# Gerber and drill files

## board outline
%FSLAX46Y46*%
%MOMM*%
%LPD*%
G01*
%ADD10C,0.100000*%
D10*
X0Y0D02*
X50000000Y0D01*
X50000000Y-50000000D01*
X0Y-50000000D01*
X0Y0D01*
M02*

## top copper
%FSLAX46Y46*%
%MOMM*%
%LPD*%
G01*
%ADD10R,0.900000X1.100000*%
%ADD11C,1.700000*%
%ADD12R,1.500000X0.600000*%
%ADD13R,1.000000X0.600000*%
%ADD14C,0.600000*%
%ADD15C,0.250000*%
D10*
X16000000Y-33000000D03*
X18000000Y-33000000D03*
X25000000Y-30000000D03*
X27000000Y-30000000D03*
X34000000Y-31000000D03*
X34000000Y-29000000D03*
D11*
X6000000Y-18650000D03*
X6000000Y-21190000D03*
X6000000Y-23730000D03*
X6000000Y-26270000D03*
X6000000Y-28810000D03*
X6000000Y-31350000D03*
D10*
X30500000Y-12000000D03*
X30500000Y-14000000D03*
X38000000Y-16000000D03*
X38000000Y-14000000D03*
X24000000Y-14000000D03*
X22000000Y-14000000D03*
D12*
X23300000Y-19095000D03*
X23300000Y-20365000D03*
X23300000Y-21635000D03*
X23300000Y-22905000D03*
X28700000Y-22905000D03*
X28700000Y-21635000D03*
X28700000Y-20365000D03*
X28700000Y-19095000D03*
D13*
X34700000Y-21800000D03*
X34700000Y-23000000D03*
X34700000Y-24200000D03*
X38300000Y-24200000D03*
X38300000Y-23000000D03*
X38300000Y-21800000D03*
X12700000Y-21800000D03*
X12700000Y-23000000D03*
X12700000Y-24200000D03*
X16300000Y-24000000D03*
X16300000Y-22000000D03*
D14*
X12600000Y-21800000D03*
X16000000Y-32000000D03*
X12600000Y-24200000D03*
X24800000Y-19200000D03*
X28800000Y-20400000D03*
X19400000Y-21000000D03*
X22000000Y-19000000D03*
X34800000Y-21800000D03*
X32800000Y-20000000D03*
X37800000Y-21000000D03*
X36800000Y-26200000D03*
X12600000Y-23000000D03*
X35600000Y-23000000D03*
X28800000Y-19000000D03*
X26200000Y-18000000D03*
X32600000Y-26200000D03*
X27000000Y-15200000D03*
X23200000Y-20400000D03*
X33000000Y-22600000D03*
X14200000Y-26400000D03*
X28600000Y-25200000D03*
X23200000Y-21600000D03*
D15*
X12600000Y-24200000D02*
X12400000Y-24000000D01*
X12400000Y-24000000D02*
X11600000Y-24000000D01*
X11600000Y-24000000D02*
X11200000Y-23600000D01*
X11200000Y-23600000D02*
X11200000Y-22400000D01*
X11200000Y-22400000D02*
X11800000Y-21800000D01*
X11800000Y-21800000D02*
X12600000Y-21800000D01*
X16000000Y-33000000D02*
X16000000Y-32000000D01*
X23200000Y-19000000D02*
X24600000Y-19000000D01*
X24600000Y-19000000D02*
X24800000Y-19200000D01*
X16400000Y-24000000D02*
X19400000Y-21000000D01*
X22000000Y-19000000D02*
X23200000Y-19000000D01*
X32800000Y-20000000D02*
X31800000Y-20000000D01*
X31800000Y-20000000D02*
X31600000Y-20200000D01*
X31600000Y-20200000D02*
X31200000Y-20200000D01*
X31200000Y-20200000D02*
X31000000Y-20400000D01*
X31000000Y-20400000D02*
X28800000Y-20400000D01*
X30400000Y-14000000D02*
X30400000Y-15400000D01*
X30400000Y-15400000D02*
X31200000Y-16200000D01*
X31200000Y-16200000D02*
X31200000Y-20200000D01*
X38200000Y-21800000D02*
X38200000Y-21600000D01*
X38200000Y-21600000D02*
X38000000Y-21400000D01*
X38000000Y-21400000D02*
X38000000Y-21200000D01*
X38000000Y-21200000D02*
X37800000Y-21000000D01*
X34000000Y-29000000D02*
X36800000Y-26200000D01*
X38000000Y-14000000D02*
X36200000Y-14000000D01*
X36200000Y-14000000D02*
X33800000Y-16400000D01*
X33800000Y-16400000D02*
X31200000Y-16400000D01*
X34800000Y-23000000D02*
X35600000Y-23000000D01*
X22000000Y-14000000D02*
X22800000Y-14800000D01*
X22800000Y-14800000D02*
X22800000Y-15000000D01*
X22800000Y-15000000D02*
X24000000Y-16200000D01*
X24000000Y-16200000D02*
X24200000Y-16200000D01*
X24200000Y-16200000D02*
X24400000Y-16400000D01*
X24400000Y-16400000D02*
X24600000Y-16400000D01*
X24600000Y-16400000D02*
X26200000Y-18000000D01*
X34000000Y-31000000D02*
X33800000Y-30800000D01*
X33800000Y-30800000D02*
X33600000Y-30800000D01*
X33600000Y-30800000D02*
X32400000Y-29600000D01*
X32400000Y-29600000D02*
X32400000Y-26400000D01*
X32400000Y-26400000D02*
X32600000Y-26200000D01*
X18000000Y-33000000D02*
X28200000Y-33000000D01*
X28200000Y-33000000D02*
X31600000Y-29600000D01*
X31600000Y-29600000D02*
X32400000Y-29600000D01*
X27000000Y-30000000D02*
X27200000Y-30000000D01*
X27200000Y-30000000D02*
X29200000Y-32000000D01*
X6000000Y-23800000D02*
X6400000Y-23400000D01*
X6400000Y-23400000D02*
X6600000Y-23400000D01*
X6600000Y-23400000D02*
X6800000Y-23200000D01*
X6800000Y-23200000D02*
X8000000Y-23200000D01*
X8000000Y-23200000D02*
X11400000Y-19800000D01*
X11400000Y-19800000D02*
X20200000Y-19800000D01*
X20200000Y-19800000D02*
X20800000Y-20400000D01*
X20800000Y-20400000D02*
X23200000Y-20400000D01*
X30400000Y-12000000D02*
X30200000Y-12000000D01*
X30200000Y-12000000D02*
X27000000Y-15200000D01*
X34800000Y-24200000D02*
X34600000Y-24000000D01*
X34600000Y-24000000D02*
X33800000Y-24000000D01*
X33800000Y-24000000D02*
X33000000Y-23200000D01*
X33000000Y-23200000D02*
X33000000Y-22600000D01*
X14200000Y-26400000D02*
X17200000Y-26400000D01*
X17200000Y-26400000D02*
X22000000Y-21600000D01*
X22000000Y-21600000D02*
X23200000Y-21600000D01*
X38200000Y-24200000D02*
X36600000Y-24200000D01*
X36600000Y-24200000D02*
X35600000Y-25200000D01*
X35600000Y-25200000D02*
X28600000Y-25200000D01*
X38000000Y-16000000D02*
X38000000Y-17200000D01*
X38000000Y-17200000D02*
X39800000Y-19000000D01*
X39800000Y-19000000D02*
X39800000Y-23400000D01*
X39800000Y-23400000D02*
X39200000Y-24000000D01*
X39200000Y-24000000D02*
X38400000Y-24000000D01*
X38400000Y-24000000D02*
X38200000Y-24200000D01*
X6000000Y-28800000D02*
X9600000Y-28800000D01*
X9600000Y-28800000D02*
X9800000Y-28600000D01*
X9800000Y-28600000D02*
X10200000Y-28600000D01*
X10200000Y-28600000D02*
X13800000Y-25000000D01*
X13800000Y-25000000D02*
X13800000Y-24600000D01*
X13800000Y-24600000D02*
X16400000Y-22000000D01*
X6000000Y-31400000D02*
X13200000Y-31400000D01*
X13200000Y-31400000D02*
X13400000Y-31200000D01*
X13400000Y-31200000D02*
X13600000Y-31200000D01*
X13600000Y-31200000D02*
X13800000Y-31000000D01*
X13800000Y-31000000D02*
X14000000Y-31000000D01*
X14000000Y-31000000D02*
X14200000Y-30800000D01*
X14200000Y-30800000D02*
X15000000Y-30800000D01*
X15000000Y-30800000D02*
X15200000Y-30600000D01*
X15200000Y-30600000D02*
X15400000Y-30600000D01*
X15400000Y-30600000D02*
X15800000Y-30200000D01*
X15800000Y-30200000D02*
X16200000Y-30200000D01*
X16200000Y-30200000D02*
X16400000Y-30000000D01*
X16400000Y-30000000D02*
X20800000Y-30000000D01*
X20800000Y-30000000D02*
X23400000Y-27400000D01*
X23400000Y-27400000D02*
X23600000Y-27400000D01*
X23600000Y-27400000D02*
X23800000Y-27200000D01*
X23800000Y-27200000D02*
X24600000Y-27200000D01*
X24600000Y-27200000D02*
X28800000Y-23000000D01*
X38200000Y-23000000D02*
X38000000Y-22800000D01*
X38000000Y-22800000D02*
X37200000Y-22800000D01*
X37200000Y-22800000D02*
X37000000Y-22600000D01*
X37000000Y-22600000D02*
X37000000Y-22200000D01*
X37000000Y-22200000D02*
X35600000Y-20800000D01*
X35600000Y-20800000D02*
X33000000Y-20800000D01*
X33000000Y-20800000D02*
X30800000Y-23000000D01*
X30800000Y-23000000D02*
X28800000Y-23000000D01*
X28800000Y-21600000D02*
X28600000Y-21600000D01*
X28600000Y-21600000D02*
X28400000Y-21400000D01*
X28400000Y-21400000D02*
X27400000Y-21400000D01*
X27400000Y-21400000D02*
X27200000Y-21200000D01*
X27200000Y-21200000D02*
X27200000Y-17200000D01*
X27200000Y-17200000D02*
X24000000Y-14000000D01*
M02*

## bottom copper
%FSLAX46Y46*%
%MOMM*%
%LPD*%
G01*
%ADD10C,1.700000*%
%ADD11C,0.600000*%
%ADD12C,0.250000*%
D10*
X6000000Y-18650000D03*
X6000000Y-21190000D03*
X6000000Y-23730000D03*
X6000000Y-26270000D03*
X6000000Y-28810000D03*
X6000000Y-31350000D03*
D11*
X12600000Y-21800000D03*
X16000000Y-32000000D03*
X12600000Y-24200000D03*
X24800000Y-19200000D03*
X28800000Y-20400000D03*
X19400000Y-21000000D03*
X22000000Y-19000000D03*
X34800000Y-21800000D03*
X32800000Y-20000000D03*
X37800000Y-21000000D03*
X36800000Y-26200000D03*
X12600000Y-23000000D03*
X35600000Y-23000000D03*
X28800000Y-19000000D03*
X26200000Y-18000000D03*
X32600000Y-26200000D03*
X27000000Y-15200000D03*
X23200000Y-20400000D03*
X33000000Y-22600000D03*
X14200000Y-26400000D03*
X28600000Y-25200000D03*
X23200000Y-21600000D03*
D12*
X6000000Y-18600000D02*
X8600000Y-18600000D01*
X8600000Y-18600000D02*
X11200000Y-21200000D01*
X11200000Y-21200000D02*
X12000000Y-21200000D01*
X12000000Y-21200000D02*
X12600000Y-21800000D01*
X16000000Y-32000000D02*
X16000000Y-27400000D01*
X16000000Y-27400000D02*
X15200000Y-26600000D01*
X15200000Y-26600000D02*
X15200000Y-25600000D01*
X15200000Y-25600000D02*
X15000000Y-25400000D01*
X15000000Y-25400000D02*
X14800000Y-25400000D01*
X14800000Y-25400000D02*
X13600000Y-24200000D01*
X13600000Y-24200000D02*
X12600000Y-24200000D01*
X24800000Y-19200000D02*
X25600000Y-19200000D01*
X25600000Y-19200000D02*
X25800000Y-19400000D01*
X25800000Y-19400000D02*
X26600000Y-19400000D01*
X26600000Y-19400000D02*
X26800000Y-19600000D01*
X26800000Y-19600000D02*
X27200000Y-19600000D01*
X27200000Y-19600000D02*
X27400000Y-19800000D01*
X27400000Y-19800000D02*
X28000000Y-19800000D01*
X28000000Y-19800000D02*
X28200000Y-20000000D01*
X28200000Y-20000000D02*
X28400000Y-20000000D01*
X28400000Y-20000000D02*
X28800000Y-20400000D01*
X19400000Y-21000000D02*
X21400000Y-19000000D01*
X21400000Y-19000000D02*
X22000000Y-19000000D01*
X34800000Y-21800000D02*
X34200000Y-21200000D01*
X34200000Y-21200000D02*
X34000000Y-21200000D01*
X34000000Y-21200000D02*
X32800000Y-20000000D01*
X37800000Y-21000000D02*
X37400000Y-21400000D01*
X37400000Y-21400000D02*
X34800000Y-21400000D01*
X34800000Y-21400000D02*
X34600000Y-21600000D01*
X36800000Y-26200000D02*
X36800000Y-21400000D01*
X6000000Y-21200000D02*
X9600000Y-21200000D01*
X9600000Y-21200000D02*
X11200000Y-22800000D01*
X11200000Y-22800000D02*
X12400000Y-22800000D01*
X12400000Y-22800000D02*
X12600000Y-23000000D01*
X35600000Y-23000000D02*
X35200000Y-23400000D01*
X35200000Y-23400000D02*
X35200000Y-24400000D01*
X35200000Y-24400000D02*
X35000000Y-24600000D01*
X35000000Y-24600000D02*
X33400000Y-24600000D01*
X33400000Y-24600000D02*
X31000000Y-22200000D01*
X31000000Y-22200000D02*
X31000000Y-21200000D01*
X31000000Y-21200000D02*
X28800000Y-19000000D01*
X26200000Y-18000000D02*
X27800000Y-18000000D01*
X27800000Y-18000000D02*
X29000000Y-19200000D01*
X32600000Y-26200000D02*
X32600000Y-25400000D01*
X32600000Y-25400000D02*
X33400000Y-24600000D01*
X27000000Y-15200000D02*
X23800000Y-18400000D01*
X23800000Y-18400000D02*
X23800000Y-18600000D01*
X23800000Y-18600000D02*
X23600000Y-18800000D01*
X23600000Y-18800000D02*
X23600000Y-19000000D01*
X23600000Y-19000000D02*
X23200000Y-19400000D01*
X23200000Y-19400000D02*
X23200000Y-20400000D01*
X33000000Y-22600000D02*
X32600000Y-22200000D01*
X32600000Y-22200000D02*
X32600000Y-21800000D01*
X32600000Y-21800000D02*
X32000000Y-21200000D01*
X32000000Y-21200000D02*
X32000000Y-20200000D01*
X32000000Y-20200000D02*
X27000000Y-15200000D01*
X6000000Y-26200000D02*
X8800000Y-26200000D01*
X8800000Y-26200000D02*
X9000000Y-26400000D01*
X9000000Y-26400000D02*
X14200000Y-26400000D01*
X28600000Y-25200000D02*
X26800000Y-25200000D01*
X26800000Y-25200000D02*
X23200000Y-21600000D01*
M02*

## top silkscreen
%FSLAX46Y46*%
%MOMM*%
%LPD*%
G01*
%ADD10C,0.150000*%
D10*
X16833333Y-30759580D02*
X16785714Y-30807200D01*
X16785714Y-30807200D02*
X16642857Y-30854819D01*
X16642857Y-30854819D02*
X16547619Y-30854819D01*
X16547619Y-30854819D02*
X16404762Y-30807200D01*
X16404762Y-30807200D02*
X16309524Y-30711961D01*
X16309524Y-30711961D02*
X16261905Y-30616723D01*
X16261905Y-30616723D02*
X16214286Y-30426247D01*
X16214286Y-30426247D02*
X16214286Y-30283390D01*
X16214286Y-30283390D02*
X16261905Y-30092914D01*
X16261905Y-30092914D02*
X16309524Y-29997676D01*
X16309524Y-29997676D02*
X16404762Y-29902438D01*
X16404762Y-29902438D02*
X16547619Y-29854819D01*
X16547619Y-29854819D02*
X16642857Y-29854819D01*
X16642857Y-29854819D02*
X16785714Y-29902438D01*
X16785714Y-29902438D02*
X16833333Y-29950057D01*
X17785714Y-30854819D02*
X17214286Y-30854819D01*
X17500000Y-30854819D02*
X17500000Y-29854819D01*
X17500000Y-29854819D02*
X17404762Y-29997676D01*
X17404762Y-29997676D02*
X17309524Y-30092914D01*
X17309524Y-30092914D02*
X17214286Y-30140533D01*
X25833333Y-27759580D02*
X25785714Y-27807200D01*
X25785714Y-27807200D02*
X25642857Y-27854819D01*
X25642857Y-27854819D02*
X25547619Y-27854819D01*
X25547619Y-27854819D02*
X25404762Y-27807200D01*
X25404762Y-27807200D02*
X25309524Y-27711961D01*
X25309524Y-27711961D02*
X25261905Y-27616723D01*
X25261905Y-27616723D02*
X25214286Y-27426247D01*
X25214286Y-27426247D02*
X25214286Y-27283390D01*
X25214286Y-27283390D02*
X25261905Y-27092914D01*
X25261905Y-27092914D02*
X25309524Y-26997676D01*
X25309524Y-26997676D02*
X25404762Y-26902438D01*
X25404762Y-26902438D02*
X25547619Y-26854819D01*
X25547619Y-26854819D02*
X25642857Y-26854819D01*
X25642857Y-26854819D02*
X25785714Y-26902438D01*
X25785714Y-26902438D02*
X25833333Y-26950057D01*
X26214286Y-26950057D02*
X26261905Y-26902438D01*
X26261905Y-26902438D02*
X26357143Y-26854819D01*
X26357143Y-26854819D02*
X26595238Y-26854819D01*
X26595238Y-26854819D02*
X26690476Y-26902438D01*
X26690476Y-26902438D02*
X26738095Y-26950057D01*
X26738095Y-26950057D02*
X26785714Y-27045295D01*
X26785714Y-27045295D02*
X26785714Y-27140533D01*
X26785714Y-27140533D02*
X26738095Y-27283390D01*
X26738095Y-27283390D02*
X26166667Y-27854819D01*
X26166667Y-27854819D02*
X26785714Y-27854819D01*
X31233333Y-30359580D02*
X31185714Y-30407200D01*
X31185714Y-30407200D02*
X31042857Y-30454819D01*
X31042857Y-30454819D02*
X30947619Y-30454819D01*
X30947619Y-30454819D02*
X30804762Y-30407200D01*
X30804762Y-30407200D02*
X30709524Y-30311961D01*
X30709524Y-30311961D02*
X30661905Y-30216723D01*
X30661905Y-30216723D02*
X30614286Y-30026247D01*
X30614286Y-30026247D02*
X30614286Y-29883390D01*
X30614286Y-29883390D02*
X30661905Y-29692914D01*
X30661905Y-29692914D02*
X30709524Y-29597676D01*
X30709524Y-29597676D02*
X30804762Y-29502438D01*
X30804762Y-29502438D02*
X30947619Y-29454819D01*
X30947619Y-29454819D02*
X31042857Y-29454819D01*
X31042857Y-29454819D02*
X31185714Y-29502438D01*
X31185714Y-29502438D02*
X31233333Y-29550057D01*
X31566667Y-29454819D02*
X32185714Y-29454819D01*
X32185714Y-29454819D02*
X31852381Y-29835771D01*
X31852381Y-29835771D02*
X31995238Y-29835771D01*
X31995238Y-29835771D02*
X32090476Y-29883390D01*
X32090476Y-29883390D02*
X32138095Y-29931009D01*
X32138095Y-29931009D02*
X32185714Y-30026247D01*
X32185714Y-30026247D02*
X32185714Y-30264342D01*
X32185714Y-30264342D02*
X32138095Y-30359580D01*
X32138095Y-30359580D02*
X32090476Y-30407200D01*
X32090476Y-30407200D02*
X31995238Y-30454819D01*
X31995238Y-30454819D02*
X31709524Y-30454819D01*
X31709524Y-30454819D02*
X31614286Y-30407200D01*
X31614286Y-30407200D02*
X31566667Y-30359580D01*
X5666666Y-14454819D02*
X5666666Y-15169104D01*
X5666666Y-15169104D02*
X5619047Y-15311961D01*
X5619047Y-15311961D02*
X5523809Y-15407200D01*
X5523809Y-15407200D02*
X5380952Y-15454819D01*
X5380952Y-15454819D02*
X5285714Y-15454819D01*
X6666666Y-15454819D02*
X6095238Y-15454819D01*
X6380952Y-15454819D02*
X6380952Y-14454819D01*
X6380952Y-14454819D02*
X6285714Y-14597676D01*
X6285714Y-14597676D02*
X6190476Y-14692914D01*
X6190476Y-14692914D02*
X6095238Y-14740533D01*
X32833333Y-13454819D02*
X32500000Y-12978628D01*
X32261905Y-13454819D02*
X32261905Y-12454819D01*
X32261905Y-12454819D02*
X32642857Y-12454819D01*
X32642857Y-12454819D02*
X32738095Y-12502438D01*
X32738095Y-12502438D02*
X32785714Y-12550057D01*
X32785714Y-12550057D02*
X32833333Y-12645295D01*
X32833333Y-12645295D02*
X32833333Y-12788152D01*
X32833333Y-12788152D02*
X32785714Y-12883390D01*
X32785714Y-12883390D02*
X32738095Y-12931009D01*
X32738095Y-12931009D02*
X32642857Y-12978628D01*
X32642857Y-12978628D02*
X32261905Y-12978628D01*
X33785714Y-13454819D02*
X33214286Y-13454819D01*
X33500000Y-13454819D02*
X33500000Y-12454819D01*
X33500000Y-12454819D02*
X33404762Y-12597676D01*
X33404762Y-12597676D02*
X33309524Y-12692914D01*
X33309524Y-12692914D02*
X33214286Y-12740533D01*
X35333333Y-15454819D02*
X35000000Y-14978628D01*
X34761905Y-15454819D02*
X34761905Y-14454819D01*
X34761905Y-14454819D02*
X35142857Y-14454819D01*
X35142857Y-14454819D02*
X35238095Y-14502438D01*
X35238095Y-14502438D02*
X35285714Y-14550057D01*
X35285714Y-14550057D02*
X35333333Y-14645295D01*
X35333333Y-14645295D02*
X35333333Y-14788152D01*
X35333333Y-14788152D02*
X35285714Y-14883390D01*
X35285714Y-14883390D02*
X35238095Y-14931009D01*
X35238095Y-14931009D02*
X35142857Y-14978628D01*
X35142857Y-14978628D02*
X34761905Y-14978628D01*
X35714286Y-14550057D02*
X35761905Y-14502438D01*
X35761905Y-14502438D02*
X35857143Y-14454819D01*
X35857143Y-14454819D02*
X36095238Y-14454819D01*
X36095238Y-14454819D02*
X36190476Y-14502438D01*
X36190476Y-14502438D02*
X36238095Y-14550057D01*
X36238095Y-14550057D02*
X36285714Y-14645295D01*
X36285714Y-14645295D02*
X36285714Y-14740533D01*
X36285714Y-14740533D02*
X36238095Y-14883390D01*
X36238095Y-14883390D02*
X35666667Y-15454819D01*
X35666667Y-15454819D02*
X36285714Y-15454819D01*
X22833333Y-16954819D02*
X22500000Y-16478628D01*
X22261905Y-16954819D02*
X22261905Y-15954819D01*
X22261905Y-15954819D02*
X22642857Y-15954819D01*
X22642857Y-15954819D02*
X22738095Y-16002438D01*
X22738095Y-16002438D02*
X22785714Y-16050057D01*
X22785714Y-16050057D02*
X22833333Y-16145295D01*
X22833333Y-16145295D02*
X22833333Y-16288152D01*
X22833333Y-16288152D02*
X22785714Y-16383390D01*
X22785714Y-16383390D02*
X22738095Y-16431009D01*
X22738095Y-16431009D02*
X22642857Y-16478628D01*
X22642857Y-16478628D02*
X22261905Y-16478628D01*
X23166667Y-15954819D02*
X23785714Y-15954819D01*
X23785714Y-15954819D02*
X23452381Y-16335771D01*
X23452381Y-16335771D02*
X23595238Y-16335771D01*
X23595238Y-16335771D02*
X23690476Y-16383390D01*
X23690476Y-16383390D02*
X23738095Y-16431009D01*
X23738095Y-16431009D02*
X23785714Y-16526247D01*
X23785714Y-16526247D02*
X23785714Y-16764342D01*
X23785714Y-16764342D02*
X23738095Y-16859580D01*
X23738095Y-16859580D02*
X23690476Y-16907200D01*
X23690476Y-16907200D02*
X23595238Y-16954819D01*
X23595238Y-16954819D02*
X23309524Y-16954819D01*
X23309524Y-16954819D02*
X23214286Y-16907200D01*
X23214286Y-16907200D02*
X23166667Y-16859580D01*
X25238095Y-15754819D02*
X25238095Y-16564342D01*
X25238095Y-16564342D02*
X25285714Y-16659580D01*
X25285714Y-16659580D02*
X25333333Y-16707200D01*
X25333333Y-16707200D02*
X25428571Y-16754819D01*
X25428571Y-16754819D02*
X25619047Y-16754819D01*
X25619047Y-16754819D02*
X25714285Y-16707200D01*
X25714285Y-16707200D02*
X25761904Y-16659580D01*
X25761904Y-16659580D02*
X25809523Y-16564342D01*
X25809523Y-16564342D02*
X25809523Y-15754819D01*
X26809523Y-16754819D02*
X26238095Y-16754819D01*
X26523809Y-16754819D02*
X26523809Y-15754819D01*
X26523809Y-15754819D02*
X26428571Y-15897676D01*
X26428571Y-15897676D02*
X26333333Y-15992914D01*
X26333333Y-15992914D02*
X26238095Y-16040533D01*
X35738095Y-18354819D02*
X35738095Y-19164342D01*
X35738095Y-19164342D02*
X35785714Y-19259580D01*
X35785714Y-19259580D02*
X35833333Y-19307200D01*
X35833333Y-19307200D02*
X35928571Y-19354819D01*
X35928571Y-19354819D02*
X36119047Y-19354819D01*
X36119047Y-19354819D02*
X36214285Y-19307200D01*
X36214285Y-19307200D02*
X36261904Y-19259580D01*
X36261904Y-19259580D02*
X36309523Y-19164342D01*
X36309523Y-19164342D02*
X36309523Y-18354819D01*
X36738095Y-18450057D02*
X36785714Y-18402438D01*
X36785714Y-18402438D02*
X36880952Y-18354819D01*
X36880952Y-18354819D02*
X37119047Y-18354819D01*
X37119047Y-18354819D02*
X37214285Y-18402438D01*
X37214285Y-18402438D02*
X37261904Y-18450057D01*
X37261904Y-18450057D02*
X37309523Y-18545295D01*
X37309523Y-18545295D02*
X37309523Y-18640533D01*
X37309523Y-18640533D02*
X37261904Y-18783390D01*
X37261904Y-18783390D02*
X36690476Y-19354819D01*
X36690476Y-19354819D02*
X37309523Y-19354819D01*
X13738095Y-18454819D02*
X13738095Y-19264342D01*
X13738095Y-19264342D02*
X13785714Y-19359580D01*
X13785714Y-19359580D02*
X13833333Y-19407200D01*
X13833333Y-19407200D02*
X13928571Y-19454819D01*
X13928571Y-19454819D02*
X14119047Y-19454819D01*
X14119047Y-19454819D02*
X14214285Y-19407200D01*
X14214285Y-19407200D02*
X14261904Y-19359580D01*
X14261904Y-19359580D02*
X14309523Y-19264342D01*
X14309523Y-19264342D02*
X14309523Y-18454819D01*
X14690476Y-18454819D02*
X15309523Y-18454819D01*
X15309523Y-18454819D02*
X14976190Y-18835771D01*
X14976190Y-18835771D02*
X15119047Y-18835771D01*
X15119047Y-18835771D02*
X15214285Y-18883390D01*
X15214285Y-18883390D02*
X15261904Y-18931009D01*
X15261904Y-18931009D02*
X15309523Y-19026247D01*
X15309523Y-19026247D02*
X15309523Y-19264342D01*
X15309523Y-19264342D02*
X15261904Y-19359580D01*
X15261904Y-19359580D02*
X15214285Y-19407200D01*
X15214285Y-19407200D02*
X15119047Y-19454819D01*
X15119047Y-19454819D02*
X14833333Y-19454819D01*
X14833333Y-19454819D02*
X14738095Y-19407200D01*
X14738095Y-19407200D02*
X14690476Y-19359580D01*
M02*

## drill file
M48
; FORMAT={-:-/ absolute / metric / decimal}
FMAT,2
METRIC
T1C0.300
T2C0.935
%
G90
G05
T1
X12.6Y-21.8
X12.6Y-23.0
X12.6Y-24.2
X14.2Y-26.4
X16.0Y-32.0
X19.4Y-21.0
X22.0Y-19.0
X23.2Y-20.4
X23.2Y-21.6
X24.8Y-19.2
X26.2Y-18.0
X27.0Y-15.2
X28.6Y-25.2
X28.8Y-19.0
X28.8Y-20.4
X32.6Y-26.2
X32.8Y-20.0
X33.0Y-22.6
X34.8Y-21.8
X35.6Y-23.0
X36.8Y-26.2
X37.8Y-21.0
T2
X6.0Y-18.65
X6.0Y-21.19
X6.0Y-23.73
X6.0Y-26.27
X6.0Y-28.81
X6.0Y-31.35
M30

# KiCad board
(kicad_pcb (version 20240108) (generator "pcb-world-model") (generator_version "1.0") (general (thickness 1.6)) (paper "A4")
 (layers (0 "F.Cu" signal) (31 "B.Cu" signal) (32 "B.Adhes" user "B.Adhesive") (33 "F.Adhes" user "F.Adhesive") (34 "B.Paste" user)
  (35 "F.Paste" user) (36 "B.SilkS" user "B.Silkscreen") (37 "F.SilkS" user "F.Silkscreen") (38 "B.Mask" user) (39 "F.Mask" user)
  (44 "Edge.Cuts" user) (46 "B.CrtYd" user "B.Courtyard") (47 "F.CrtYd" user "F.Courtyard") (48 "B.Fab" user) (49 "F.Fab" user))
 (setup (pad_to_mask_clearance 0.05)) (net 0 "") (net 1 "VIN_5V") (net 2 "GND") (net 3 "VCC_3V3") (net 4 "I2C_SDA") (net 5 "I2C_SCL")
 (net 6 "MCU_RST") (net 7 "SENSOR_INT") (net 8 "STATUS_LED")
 (gr_rect (start 0.0 0.0) (end 50.0000 50.0000) (stroke (width 0.1) (type default)) (fill none) (layer "Edge.Cuts"))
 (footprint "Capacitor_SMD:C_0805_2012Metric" (layer "F.Cu") (at 17.0000 33.0000 0)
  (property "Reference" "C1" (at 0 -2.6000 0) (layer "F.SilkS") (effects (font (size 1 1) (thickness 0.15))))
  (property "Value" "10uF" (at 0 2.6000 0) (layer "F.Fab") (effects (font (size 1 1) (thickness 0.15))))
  (pad "1" smd rect (at -1.0000 0.0000) (size 0.9000 1.1000) (layers "F.Cu" "F.Paste" "F.Mask") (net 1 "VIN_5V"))
  (pad "2" smd rect (at 1.0000 0.0000) (size 0.9000 1.1000) (layers "F.Cu" "F.Paste" "F.Mask") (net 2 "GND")))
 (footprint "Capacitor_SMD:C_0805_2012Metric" (layer "F.Cu") (at 26.0000 30.0000 0)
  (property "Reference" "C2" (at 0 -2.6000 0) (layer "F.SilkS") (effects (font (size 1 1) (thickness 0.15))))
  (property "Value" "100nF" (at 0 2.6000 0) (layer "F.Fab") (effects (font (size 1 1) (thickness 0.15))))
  (pad "1" smd rect (at -1.0000 0.0000) (size 0.9000 1.1000) (layers "F.Cu" "F.Paste" "F.Mask") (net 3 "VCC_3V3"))
  (pad "2" smd rect (at 1.0000 0.0000) (size 0.9000 1.1000) (layers "F.Cu" "F.Paste" "F.Mask") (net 2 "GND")))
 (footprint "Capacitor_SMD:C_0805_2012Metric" (layer "F.Cu") (at 34.0000 30.0000 90)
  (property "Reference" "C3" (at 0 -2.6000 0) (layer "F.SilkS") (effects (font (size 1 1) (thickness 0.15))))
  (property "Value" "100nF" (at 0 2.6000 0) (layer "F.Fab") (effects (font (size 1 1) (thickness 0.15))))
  (pad "1" smd rect (at -1.0000 0.0000) (size 0.9000 1.1000) (layers "F.Cu" "F.Paste" "F.Mask") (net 3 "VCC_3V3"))
  (pad "2" smd rect (at 1.0000 0.0000) (size 0.9000 1.1000) (layers "F.Cu" "F.Paste" "F.Mask") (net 2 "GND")))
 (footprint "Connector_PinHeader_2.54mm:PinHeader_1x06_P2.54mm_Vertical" (layer "F.Cu") (at 6.0000 25.0000 0) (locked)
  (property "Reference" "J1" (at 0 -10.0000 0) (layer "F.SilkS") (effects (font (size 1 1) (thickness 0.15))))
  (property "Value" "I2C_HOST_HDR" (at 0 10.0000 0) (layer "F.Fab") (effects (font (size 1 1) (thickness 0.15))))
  (pad "1" thru_hole circle (at 0.0000 -6.3500) (size 1.7000 1.7000) (drill 0.9350) (layers "*.Cu" "*.Mask") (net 1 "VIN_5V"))
  (pad "2" thru_hole circle (at 0.0000 -3.8100) (size 1.7000 1.7000) (drill 0.9350) (layers "*.Cu" "*.Mask") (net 2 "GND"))
  (pad "3" thru_hole circle (at 0.0000 -1.2700) (size 1.7000 1.7000) (drill 0.9350) (layers "*.Cu" "*.Mask") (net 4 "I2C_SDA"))
  (pad "4" thru_hole circle (at 0.0000 1.2700) (size 1.7000 1.7000) (drill 0.9350) (layers "*.Cu" "*.Mask") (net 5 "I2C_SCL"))
  (pad "5" thru_hole circle (at 0.0000 3.8100) (size 1.7000 1.7000) (drill 0.9350) (layers "*.Cu" "*.Mask") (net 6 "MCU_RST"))
  (pad "6" thru_hole circle (at 0.0000 6.3500) (size 1.7000 1.7000) (drill 0.9350) (layers "*.Cu" "*.Mask") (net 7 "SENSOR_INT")))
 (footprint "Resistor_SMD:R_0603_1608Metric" (layer "F.Cu") (at 30.5000 13.0000 270)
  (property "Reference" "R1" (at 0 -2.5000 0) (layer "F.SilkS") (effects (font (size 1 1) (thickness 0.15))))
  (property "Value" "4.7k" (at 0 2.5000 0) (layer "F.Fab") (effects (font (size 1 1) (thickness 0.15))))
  (pad "1" smd rect (at -1.0000 0.0000) (size 0.9000 1.1000) (layers "F.Cu" "F.Paste" "F.Mask") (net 3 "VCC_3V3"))
  (pad "2" smd rect (at 1.0000 0.0000) (size 0.9000 1.1000) (layers "F.Cu" "F.Paste" "F.Mask") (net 4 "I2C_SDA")))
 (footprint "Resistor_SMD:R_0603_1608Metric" (layer "F.Cu") (at 38.0000 15.0000 90)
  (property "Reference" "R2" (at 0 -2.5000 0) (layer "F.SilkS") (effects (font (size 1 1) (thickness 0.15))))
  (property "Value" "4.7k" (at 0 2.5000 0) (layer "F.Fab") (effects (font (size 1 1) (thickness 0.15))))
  (pad "1" smd rect (at -1.0000 0.0000) (size 0.9000 1.1000) (layers "F.Cu" "F.Paste" "F.Mask") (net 3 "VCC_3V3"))
  (pad "2" smd rect (at 1.0000 0.0000) (size 0.9000 1.1000) (layers "F.Cu" "F.Paste" "F.Mask") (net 5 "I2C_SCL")))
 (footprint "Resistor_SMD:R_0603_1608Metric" (layer "F.Cu") (at 23.0000 14.0000 180)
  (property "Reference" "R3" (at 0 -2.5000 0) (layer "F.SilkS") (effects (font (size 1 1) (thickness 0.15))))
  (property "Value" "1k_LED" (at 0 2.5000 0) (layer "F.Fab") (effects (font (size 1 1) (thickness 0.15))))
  (pad "1" smd rect (at -1.0000 0.0000) (size 0.9000 1.1000) (layers "F.Cu" "F.Paste" "F.Mask") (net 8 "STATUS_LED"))
  (pad "2" smd rect (at 1.0000 0.0000) (size 0.9000 1.1000) (layers "F.Cu" "F.Paste" "F.Mask") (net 2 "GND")))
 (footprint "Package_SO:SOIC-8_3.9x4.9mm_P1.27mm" (layer "F.Cu") (at 26.0000 21.0000 0)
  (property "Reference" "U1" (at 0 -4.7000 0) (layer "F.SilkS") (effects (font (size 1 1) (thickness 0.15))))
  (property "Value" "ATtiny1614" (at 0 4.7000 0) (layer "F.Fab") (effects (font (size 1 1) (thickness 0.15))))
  (pad "1" smd rect (at -2.7000 -1.9050) (size 1.5000 0.6000) (layers "F.Cu" "F.Paste" "F.Mask") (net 3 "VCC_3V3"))
  (pad "2" smd rect (at -2.7000 -0.6350) (size 1.5000 0.6000) (layers "F.Cu" "F.Paste" "F.Mask") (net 4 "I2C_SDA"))
  (pad "3" smd rect (at -2.7000 0.6350) (size 1.5000 0.6000) (layers "F.Cu" "F.Paste" "F.Mask") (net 5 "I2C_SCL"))
  (pad "4" smd rect (at -2.7000 1.9050) (size 1.5000 0.6000) (layers "F.Cu" "F.Paste" "F.Mask") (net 6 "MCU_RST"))
  (pad "5" smd rect (at 2.7000 1.9050) (size 1.5000 0.6000) (layers "F.Cu" "F.Paste" "F.Mask") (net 7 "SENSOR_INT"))
  (pad "6" smd rect (at 2.7000 0.6350) (size 1.5000 0.6000) (layers "F.Cu" "F.Paste" "F.Mask") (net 8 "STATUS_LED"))
  (pad "7" smd rect (at 2.7000 -0.6350) (size 1.5000 0.6000) (layers "F.Cu" "F.Paste" "F.Mask") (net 3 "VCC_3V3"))
  (pad "8" smd rect (at 2.7000 -1.9050) (size 1.5000 0.6000) (layers "F.Cu" "F.Paste" "F.Mask") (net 2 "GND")))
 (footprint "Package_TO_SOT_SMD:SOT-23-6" (layer "F.Cu") (at 36.5000 23.0000 0)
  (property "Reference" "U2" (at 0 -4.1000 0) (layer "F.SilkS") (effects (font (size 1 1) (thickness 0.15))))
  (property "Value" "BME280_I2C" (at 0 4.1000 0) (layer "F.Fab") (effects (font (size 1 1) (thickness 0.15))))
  (pad "1" smd rect (at -1.8000 -1.2000) (size 1.0000 0.6000) (layers "F.Cu" "F.Paste" "F.Mask") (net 3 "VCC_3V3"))
  (pad "2" smd rect (at -1.8000 0.0000) (size 1.0000 0.6000) (layers "F.Cu" "F.Paste" "F.Mask") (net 2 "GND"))
  (pad "3" smd rect (at -1.8000 1.2000) (size 1.0000 0.6000) (layers "F.Cu" "F.Paste" "F.Mask") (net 4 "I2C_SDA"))
  (pad "4" smd rect (at 1.8000 1.2000) (size 1.0000 0.6000) (layers "F.Cu" "F.Paste" "F.Mask") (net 5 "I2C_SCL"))
  (pad "5" smd rect (at 1.8000 0.0000) (size 1.0000 0.6000) (layers "F.Cu" "F.Paste" "F.Mask") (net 7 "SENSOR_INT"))
  (pad "6" smd rect (at 1.8000 -1.2000) (size 1.0000 0.6000) (layers "F.Cu" "F.Paste" "F.Mask") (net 3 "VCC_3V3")))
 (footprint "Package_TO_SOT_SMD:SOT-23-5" (layer "F.Cu") (at 14.5000 23.0000 0)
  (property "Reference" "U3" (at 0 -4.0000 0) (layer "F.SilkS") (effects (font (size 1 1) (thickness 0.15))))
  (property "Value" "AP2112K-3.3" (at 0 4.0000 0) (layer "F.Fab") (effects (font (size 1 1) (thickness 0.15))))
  (pad "1" smd rect (at -1.8000 -1.2000) (size 1.0000 0.6000) (layers "F.Cu" "F.Paste" "F.Mask") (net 1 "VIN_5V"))
  (pad "2" smd rect (at -1.8000 0.0000) (size 1.0000 0.6000) (layers "F.Cu" "F.Paste" "F.Mask") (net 2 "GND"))
  (pad "3" smd rect (at -1.8000 1.2000) (size 1.0000 0.6000) (layers "F.Cu" "F.Paste" "F.Mask") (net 1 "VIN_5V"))
  (pad "4" smd rect (at 1.8000 1.0000) (size 1.0000 0.6000) (layers "F.Cu" "F.Paste" "F.Mask") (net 3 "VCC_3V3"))
  (pad "5" smd rect (at 1.8000 -1.0000) (size 1.0000 0.6000) (layers "F.Cu" "F.Paste" "F.Mask") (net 6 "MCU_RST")))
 (segment (start 6.0000 18.6000) (end 8.6000 18.6000) (width 0.2500) (layer "B.Cu") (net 1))
 (segment (start 8.6000 18.6000) (end 11.2000 21.2000) (width 0.2500) (layer "B.Cu") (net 1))
 (segment (start 11.2000 21.2000) (end 12.0000 21.2000) (width 0.2500) (layer "B.Cu") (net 1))
 (segment (start 12.0000 21.2000) (end 12.6000 21.8000) (width 0.2500) (layer "B.Cu") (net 1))
 (segment (start 12.6000 24.2000) (end 12.4000 24.0000) (width 0.2500) (layer "F.Cu") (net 1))
 (segment (start 12.4000 24.0000) (end 11.6000 24.0000) (width 0.2500) (layer "F.Cu") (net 1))
 (segment (start 11.6000 24.0000) (end 11.2000 23.6000) (width 0.2500) (layer "F.Cu") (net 1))
 (segment (start 11.2000 23.6000) (end 11.2000 22.4000) (width 0.2500) (layer "F.Cu") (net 1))
 (segment (start 11.2000 22.4000) (end 11.8000 21.8000) (width 0.2500) (layer "F.Cu") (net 1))
 (segment (start 11.8000 21.8000) (end 12.6000 21.8000) (width 0.2500) (layer "F.Cu") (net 1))
 (segment (start 16.0000 33.0000) (end 16.0000 32.0000) (width 0.2500) (layer "F.Cu") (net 1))
 (segment (start 16.0000 32.0000) (end 16.0000 27.4000) (width 0.2500) (layer "B.Cu") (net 1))
 (segment (start 16.0000 27.4000) (end 15.2000 26.6000) (width 0.2500) (layer "B.Cu") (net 1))
 (segment (start 15.2000 26.6000) (end 15.2000 25.6000) (width 0.2500) (layer "B.Cu") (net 1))
 (segment (start 15.2000 25.6000) (end 15.0000 25.4000) (width 0.2500) (layer "B.Cu") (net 1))
 (segment (start 15.0000 25.4000) (end 14.8000 25.4000) (width 0.2500) (layer "B.Cu") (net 1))
 (segment (start 14.8000 25.4000) (end 13.6000 24.2000) (width 0.2500) (layer "B.Cu") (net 1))
 (segment (start 13.6000 24.2000) (end 12.6000 24.2000) (width 0.2500) (layer "B.Cu") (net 1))
 (segment (start 23.2000 19.0000) (end 24.6000 19.0000) (width 0.2500) (layer "F.Cu") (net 3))
 (segment (start 24.6000 19.0000) (end 24.8000 19.2000) (width 0.2500) (layer "F.Cu") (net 3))
 (segment (start 24.8000 19.2000) (end 25.6000 19.2000) (width 0.2500) (layer "B.Cu") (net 3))
 (segment (start 25.6000 19.2000) (end 25.8000 19.4000) (width 0.2500) (layer "B.Cu") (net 3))
 (segment (start 25.8000 19.4000) (end 26.6000 19.4000) (width 0.2500) (layer "B.Cu") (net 3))
 (segment (start 26.6000 19.4000) (end 26.8000 19.6000) (width 0.2500) (layer "B.Cu") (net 3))
 (segment (start 26.8000 19.6000) (end 27.2000 19.6000) (width 0.2500) (layer "B.Cu") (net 3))
 (segment (start 27.2000 19.6000) (end 27.4000 19.8000) (width 0.2500) (layer "B.Cu") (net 3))
 (segment (start 27.4000 19.8000) (end 28.0000 19.8000) (width 0.2500) (layer "B.Cu") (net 3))
 (segment (start 28.0000 19.8000) (end 28.2000 20.0000) (width 0.2500) (layer "B.Cu") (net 3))
 (segment (start 28.2000 20.0000) (end 28.4000 20.0000) (width 0.2500) (layer "B.Cu") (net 3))
 (segment (start 28.4000 20.0000) (end 28.8000 20.4000) (width 0.2500) (layer "B.Cu") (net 3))
 (segment (start 16.4000 24.0000) (end 19.4000 21.0000) (width 0.2500) (layer "F.Cu") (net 3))
 (segment (start 19.4000 21.0000) (end 21.4000 19.0000) (width 0.2500) (layer "B.Cu") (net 3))
 (segment (start 21.4000 19.0000) (end 22.0000 19.0000) (width 0.2500) (layer "B.Cu") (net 3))
 (segment (start 22.0000 19.0000) (end 23.2000 19.0000) (width 0.2500) (layer "F.Cu") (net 3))
 (segment (start 34.8000 21.8000) (end 34.2000 21.2000) (width 0.2500) (layer "B.Cu") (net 3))
 (segment (start 34.2000 21.2000) (end 34.0000 21.2000) (width 0.2500) (layer "B.Cu") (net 3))
 (segment (start 34.0000 21.2000) (end 32.8000 20.0000) (width 0.2500) (layer "B.Cu") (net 3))
 (segment (start 32.8000 20.0000) (end 31.8000 20.0000) (width 0.2500) (layer "F.Cu") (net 3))
 (segment (start 31.8000 20.0000) (end 31.6000 20.2000) (width 0.2500) (layer "F.Cu") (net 3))
 (segment (start 31.6000 20.2000) (end 31.2000 20.2000) (width 0.2500) (layer "F.Cu") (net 3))
 (segment (start 31.2000 20.2000) (end 31.0000 20.4000) (width 0.2500) (layer "F.Cu") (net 3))
 (segment (start 31.0000 20.4000) (end 28.8000 20.4000) (width 0.2500) (layer "F.Cu") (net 3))
 (segment (start 30.4000 14.0000) (end 30.4000 15.4000) (width 0.2500) (layer "F.Cu") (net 3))
 (segment (start 30.4000 15.4000) (end 31.2000 16.2000) (width 0.2500) (layer "F.Cu") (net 3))
 (segment (start 31.2000 16.2000) (end 31.2000 20.2000) (width 0.2500) (layer "F.Cu") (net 3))
 (segment (start 38.2000 21.8000) (end 38.2000 21.6000) (width 0.2500) (layer "F.Cu") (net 3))
 (segment (start 38.2000 21.6000) (end 38.0000 21.4000) (width 0.2500) (layer "F.Cu") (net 3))
 (segment (start 38.0000 21.4000) (end 38.0000 21.2000) (width 0.2500) (layer "F.Cu") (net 3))
 (segment (start 38.0000 21.2000) (end 37.8000 21.0000) (width 0.2500) (layer "F.Cu") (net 3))
 (segment (start 37.8000 21.0000) (end 37.4000 21.4000) (width 0.2500) (layer "B.Cu") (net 3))
 (segment (start 37.4000 21.4000) (end 34.8000 21.4000) (width 0.2500) (layer "B.Cu") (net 3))
 (segment (start 34.8000 21.4000) (end 34.6000 21.6000) (width 0.2500) (layer "B.Cu") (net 3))
 (segment (start 34.0000 29.0000) (end 36.8000 26.2000) (width 0.2500) (layer "F.Cu") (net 3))
 (segment (start 36.8000 26.2000) (end 36.8000 21.4000) (width 0.2500) (layer "B.Cu") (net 3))
 (segment (start 38.0000 14.0000) (end 36.2000 14.0000) (width 0.2500) (layer "F.Cu") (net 3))
 (segment (start 36.2000 14.0000) (end 33.8000 16.4000) (width 0.2500) (layer "F.Cu") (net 3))
 (segment (start 33.8000 16.4000) (end 31.2000 16.4000) (width 0.2500) (layer "F.Cu") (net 3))
 (segment (start 6.0000 21.2000) (end 9.6000 21.2000) (width 0.2500) (layer "B.Cu") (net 2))
 (segment (start 9.6000 21.2000) (end 11.2000 22.8000) (width 0.2500) (layer "B.Cu") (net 2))
 (segment (start 11.2000 22.8000) (end 12.4000 22.8000) (width 0.2500) (layer "B.Cu") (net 2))
 (segment (start 12.4000 22.8000) (end 12.6000 23.0000) (width 0.2500) (layer "B.Cu") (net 2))
 (segment (start 34.8000 23.0000) (end 35.6000 23.0000) (width 0.2500) (layer "F.Cu") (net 2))
 (segment (start 35.6000 23.0000) (end 35.2000 23.4000) (width 0.2500) (layer "B.Cu") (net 2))
 (segment (start 35.2000 23.4000) (end 35.2000 24.4000) (width 0.2500) (layer "B.Cu") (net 2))
 (segment (start 35.2000 24.4000) (end 35.0000 24.6000) (width 0.2500) (layer "B.Cu") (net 2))
 (segment (start 35.0000 24.6000) (end 33.4000 24.6000) (width 0.2500) (layer "B.Cu") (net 2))
 (segment (start 33.4000 24.6000) (end 31.0000 22.2000) (width 0.2500) (layer "B.Cu") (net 2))
 (segment (start 31.0000 22.2000) (end 31.0000 21.2000) (width 0.2500) (layer "B.Cu") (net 2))
 (segment (start 31.0000 21.2000) (end 28.8000 19.0000) (width 0.2500) (layer "B.Cu") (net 2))
 (segment (start 22.0000 14.0000) (end 22.8000 14.8000) (width 0.2500) (layer "F.Cu") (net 2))
 (segment (start 22.8000 14.8000) (end 22.8000 15.0000) (width 0.2500) (layer "F.Cu") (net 2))
 (segment (start 22.8000 15.0000) (end 24.0000 16.2000) (width 0.2500) (layer "F.Cu") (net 2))
 (segment (start 24.0000 16.2000) (end 24.2000 16.2000) (width 0.2500) (layer "F.Cu") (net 2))
 (segment (start 24.2000 16.2000) (end 24.4000 16.4000) (width 0.2500) (layer "F.Cu") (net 2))
 (segment (start 24.4000 16.4000) (end 24.6000 16.4000) (width 0.2500) (layer "F.Cu") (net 2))
 (segment (start 24.6000 16.4000) (end 26.2000 18.0000) (width 0.2500) (layer "F.Cu") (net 2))
 (segment (start 26.2000 18.0000) (end 27.8000 18.0000) (width 0.2500) (layer "B.Cu") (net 2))
 (segment (start 27.8000 18.0000) (end 29.0000 19.2000) (width 0.2500) (layer "B.Cu") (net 2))
 (segment (start 34.0000 31.0000) (end 33.8000 30.8000) (width 0.2500) (layer "F.Cu") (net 2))
 (segment (start 33.8000 30.8000) (end 33.6000 30.8000) (width 0.2500) (layer "F.Cu") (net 2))
 (segment (start 33.6000 30.8000) (end 32.4000 29.6000) (width 0.2500) (layer "F.Cu") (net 2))
 (segment (start 32.4000 29.6000) (end 32.4000 26.4000) (width 0.2500) (layer "F.Cu") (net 2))
 (segment (start 32.4000 26.4000) (end 32.6000 26.2000) (width 0.2500) (layer "F.Cu") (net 2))
 (segment (start 32.6000 26.2000) (end 32.6000 25.4000) (width 0.2500) (layer "B.Cu") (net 2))
 (segment (start 32.6000 25.4000) (end 33.4000 24.6000) (width 0.2500) (layer "B.Cu") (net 2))
 (segment (start 18.0000 33.0000) (end 28.2000 33.0000) (width 0.2500) (layer "F.Cu") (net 2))
 (segment (start 28.2000 33.0000) (end 31.6000 29.6000) (width 0.2500) (layer "F.Cu") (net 2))
 (segment (start 31.6000 29.6000) (end 32.4000 29.6000) (width 0.2500) (layer "F.Cu") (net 2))
 (segment (start 27.0000 30.0000) (end 27.2000 30.0000) (width 0.2500) (layer "F.Cu") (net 2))
 (segment (start 27.2000 30.0000) (end 29.2000 32.0000) (width 0.2500) (layer "F.Cu") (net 2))
 (segment (start 6.0000 23.8000) (end 6.4000 23.4000) (width 0.2500) (layer "F.Cu") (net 4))
 (segment (start 6.4000 23.4000) (end 6.6000 23.4000) (width 0.2500) (layer "F.Cu") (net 4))
 (segment (start 6.6000 23.4000) (end 6.8000 23.2000) (width 0.2500) (layer "F.Cu") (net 4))
 (segment (start 6.8000 23.2000) (end 8.0000 23.2000) (width 0.2500) (layer "F.Cu") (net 4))
 (segment (start 8.0000 23.2000) (end 11.4000 19.8000) (width 0.2500) (layer "F.Cu") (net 4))
 (segment (start 11.4000 19.8000) (end 20.2000 19.8000) (width 0.2500) (layer "F.Cu") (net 4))
 (segment (start 20.2000 19.8000) (end 20.8000 20.4000) (width 0.2500) (layer "F.Cu") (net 4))
 (segment (start 20.8000 20.4000) (end 23.2000 20.4000) (width 0.2500) (layer "F.Cu") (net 4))
 (segment (start 30.4000 12.0000) (end 30.2000 12.0000) (width 0.2500) (layer "F.Cu") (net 4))
 (segment (start 30.2000 12.0000) (end 27.0000 15.2000) (width 0.2500) (layer "F.Cu") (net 4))
 (segment (start 27.0000 15.2000) (end 23.8000 18.4000) (width 0.2500) (layer "B.Cu") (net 4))
 (segment (start 23.8000 18.4000) (end 23.8000 18.6000) (width 0.2500) (layer "B.Cu") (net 4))
 (segment (start 23.8000 18.6000) (end 23.6000 18.8000) (width 0.2500) (layer "B.Cu") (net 4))
 (segment (start 23.6000 18.8000) (end 23.6000 19.0000) (width 0.2500) (layer "B.Cu") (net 4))
 (segment (start 23.6000 19.0000) (end 23.2000 19.4000) (width 0.2500) (layer "B.Cu") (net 4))
 (segment (start 23.2000 19.4000) (end 23.2000 20.4000) (width 0.2500) (layer "B.Cu") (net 4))
 (segment (start 34.8000 24.2000) (end 34.6000 24.0000) (width 0.2500) (layer "F.Cu") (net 4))
 (segment (start 34.6000 24.0000) (end 33.8000 24.0000) (width 0.2500) (layer "F.Cu") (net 4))
 (segment (start 33.8000 24.0000) (end 33.0000 23.2000) (width 0.2500) (layer "F.Cu") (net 4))
 (segment (start 33.0000 23.2000) (end 33.0000 22.6000) (width 0.2500) (layer "F.Cu") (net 4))
 (segment (start 33.0000 22.6000) (end 32.6000 22.2000) (width 0.2500) (layer "B.Cu") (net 4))
 (segment (start 32.6000 22.2000) (end 32.6000 21.8000) (width 0.2500) (layer "B.Cu") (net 4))
 (segment (start 32.6000 21.8000) (end 32.0000 21.2000) (width 0.2500) (layer "B.Cu") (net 4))
 (segment (start 32.0000 21.2000) (end 32.0000 20.2000) (width 0.2500) (layer "B.Cu") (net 4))
 (segment (start 32.0000 20.2000) (end 27.0000 15.2000) (width 0.2500) (layer "B.Cu") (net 4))
 (segment (start 6.0000 26.2000) (end 8.8000 26.2000) (width 0.2500) (layer "B.Cu") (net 5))
 (segment (start 8.8000 26.2000) (end 9.0000 26.4000) (width 0.2500) (layer "B.Cu") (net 5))
 (segment (start 9.0000 26.4000) (end 14.2000 26.4000) (width 0.2500) (layer "B.Cu") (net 5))
 (segment (start 14.2000 26.4000) (end 17.2000 26.4000) (width 0.2500) (layer "F.Cu") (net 5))
 (segment (start 17.2000 26.4000) (end 22.0000 21.6000) (width 0.2500) (layer "F.Cu") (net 5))
 (segment (start 22.0000 21.6000) (end 23.2000 21.6000) (width 0.2500) (layer "F.Cu") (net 5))
 (segment (start 38.2000 24.2000) (end 36.6000 24.2000) (width 0.2500) (layer "F.Cu") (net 5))
 (segment (start 36.6000 24.2000) (end 35.6000 25.2000) (width 0.2500) (layer "F.Cu") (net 5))
 (segment (start 35.6000 25.2000) (end 28.6000 25.2000) (width 0.2500) (layer "F.Cu") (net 5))
 (segment (start 28.6000 25.2000) (end 26.8000 25.2000) (width 0.2500) (layer "B.Cu") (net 5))
 (segment (start 26.8000 25.2000) (end 23.2000 21.6000) (width 0.2500) (layer "B.Cu") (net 5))
 (segment (start 38.0000 16.0000) (end 38.0000 17.2000) (width 0.2500) (layer "F.Cu") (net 5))
 (segment (start 38.0000 17.2000) (end 39.8000 19.0000) (width 0.2500) (layer "F.Cu") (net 5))
 (segment (start 39.8000 19.0000) (end 39.8000 23.4000) (width 0.2500) (layer "F.Cu") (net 5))
 (segment (start 39.8000 23.4000) (end 39.2000 24.0000) (width 0.2500) (layer "F.Cu") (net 5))
 (segment (start 39.2000 24.0000) (end 38.4000 24.0000) (width 0.2500) (layer "F.Cu") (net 5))
 (segment (start 38.4000 24.0000) (end 38.2000 24.2000) (width 0.2500) (layer "F.Cu") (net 5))
 (segment (start 6.0000 28.8000) (end 9.6000 28.8000) (width 0.2500) (layer "F.Cu") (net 6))
 (segment (start 9.6000 28.8000) (end 9.8000 28.6000) (width 0.2500) (layer "F.Cu") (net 6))
 (segment (start 9.8000 28.6000) (end 10.2000 28.6000) (width 0.2500) (layer "F.Cu") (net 6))
 (segment (start 10.2000 28.6000) (end 13.8000 25.0000) (width 0.2500) (layer "F.Cu") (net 6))
 (segment (start 13.8000 25.0000) (end 13.8000 24.6000) (width 0.2500) (layer "F.Cu") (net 6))
 (segment (start 13.8000 24.6000) (end 16.4000 22.0000) (width 0.2500) (layer "F.Cu") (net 6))
 (segment (start 6.0000 31.4000) (end 13.2000 31.4000) (width 0.2500) (layer "F.Cu") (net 7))
 (segment (start 13.2000 31.4000) (end 13.4000 31.2000) (width 0.2500) (layer "F.Cu") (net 7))
 (segment (start 13.4000 31.2000) (end 13.6000 31.2000) (width 0.2500) (layer "F.Cu") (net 7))
 (segment (start 13.6000 31.2000) (end 13.8000 31.0000) (width 0.2500) (layer "F.Cu") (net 7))
 (segment (start 13.8000 31.0000) (end 14.0000 31.0000) (width 0.2500) (layer "F.Cu") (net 7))
 (segment (start 14.0000 31.0000) (end 14.2000 30.8000) (width 0.2500) (layer "F.Cu") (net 7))
 (segment (start 14.2000 30.8000) (end 15.0000 30.8000) (width 0.2500) (layer "F.Cu") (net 7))
 (segment (start 15.0000 30.8000) (end 15.2000 30.6000) (width 0.2500) (layer "F.Cu") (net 7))
 (segment (start 15.2000 30.6000) (end 15.4000 30.6000) (width 0.2500) (layer "F.Cu") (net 7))
 (segment (start 15.4000 30.6000) (end 15.8000 30.2000) (width 0.2500) (layer "F.Cu") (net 7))
 (segment (start 15.8000 30.2000) (end 16.2000 30.2000) (width 0.2500) (layer "F.Cu") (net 7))
 (segment (start 16.2000 30.2000) (end 16.4000 30.0000) (width 0.2500) (layer "F.Cu") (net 7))
 (segment (start 16.4000 30.0000) (end 20.8000 30.0000) (width 0.2500) (layer "F.Cu") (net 7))
 (segment (start 20.8000 30.0000) (end 23.4000 27.4000) (width 0.2500) (layer "F.Cu") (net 7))
 (segment (start 23.4000 27.4000) (end 23.6000 27.4000) (width 0.2500) (layer "F.Cu") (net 7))
 (segment (start 23.6000 27.4000) (end 23.8000 27.2000) (width 0.2500) (layer "F.Cu") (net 7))
 (segment (start 23.8000 27.2000) (end 24.6000 27.2000) (width 0.2500) (layer "F.Cu") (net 7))
 (segment (start 24.6000 27.2000) (end 28.8000 23.0000) (width 0.2500) (layer "F.Cu") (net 7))
 (segment (start 38.2000 23.0000) (end 38.0000 22.8000) (width 0.2500) (layer "F.Cu") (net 7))
 (segment (start 38.0000 22.8000) (end 37.2000 22.8000) (width 0.2500) (layer "F.Cu") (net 7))
 (segment (start 37.2000 22.8000) (end 37.0000 22.6000) (width 0.2500) (layer "F.Cu") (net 7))
 (segment (start 37.0000 22.6000) (end 37.0000 22.2000) (width 0.2500) (layer "F.Cu") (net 7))
 (segment (start 37.0000 22.2000) (end 35.6000 20.8000) (width 0.2500) (layer "F.Cu") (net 7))
 (segment (start 35.6000 20.8000) (end 33.0000 20.8000) (width 0.2500) (layer "F.Cu") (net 7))
 (segment (start 33.0000 20.8000) (end 30.8000 23.0000) (width 0.2500) (layer "F.Cu") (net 7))
 (segment (start 30.8000 23.0000) (end 28.8000 23.0000) (width 0.2500) (layer "F.Cu") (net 7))
 (segment (start 28.8000 21.6000) (end 28.6000 21.6000) (width 0.2500) (layer "F.Cu") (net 8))
 (segment (start 28.6000 21.6000) (end 28.4000 21.4000) (width 0.2500) (layer "F.Cu") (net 8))
 (segment (start 28.4000 21.4000) (end 27.4000 21.4000) (width 0.2500) (layer "F.Cu") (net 8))
 (segment (start 27.4000 21.4000) (end 27.2000 21.2000) (width 0.2500) (layer "F.Cu") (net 8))
 (segment (start 27.2000 21.2000) (end 27.2000 17.2000) (width 0.2500) (layer "F.Cu") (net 8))
 (segment (start 27.2000 17.2000) (end 24.0000 14.0000) (width 0.2500) (layer "F.Cu") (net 8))
 (via (at 12.6000 21.8000) (size 0.6000) (drill 0.3000) (layers "F.Cu" "B.Cu") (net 1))
 (via (at 16.0000 32.0000) (size 0.6000) (drill 0.3000) (layers "F.Cu" "B.Cu") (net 1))
 (via (at 12.6000 24.2000) (size 0.6000) (drill 0.3000) (layers "F.Cu" "B.Cu") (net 1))
 (via (at 24.8000 19.2000) (size 0.6000) (drill 0.3000) (layers "F.Cu" "B.Cu") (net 3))
 (via (at 28.8000 20.4000) (size 0.6000) (drill 0.3000) (layers "F.Cu" "B.Cu") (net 3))
 (via (at 19.4000 21.0000) (size 0.6000) (drill 0.3000) (layers "F.Cu" "B.Cu") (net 3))
 (via (at 22.0000 19.0000) (size 0.6000) (drill 0.3000) (layers "F.Cu" "B.Cu") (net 3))
 (via (at 34.8000 21.8000) (size 0.6000) (drill 0.3000) (layers "F.Cu" "B.Cu") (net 3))
 (via (at 32.8000 20.0000) (size 0.6000) (drill 0.3000) (layers "F.Cu" "B.Cu") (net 3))
 (via (at 37.8000 21.0000) (size 0.6000) (drill 0.3000) (layers "F.Cu" "B.Cu") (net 3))
 (via (at 36.8000 26.2000) (size 0.6000) (drill 0.3000) (layers "F.Cu" "B.Cu") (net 3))
 (via (at 12.6000 23.0000) (size 0.6000) (drill 0.3000) (layers "F.Cu" "B.Cu") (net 2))
 (via (at 35.6000 23.0000) (size 0.6000) (drill 0.3000) (layers "F.Cu" "B.Cu") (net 2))
 (via (at 28.8000 19.0000) (size 0.6000) (drill 0.3000) (layers "F.Cu" "B.Cu") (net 2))
 (via (at 26.2000 18.0000) (size 0.6000) (drill 0.3000) (layers "F.Cu" "B.Cu") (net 2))
 (via (at 32.6000 26.2000) (size 0.6000) (drill 0.3000) (layers "F.Cu" "B.Cu") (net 2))
 (via (at 27.0000 15.2000) (size 0.6000) (drill 0.3000) (layers "F.Cu" "B.Cu") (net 4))
 (via (at 23.2000 20.4000) (size 0.6000) (drill 0.3000) (layers "F.Cu" "B.Cu") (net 4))
 (via (at 33.0000 22.6000) (size 0.6000) (drill 0.3000) (layers "F.Cu" "B.Cu") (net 4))
 (via (at 14.2000 26.4000) (size 0.6000) (drill 0.3000) (layers "F.Cu" "B.Cu") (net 5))
 (via (at 28.6000 25.2000) (size 0.6000) (drill 0.3000) (layers "F.Cu" "B.Cu") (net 5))
 (via (at 23.2000 21.6000) (size 0.6000) (drill 0.3000) (layers "F.Cu" "B.Cu") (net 5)))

